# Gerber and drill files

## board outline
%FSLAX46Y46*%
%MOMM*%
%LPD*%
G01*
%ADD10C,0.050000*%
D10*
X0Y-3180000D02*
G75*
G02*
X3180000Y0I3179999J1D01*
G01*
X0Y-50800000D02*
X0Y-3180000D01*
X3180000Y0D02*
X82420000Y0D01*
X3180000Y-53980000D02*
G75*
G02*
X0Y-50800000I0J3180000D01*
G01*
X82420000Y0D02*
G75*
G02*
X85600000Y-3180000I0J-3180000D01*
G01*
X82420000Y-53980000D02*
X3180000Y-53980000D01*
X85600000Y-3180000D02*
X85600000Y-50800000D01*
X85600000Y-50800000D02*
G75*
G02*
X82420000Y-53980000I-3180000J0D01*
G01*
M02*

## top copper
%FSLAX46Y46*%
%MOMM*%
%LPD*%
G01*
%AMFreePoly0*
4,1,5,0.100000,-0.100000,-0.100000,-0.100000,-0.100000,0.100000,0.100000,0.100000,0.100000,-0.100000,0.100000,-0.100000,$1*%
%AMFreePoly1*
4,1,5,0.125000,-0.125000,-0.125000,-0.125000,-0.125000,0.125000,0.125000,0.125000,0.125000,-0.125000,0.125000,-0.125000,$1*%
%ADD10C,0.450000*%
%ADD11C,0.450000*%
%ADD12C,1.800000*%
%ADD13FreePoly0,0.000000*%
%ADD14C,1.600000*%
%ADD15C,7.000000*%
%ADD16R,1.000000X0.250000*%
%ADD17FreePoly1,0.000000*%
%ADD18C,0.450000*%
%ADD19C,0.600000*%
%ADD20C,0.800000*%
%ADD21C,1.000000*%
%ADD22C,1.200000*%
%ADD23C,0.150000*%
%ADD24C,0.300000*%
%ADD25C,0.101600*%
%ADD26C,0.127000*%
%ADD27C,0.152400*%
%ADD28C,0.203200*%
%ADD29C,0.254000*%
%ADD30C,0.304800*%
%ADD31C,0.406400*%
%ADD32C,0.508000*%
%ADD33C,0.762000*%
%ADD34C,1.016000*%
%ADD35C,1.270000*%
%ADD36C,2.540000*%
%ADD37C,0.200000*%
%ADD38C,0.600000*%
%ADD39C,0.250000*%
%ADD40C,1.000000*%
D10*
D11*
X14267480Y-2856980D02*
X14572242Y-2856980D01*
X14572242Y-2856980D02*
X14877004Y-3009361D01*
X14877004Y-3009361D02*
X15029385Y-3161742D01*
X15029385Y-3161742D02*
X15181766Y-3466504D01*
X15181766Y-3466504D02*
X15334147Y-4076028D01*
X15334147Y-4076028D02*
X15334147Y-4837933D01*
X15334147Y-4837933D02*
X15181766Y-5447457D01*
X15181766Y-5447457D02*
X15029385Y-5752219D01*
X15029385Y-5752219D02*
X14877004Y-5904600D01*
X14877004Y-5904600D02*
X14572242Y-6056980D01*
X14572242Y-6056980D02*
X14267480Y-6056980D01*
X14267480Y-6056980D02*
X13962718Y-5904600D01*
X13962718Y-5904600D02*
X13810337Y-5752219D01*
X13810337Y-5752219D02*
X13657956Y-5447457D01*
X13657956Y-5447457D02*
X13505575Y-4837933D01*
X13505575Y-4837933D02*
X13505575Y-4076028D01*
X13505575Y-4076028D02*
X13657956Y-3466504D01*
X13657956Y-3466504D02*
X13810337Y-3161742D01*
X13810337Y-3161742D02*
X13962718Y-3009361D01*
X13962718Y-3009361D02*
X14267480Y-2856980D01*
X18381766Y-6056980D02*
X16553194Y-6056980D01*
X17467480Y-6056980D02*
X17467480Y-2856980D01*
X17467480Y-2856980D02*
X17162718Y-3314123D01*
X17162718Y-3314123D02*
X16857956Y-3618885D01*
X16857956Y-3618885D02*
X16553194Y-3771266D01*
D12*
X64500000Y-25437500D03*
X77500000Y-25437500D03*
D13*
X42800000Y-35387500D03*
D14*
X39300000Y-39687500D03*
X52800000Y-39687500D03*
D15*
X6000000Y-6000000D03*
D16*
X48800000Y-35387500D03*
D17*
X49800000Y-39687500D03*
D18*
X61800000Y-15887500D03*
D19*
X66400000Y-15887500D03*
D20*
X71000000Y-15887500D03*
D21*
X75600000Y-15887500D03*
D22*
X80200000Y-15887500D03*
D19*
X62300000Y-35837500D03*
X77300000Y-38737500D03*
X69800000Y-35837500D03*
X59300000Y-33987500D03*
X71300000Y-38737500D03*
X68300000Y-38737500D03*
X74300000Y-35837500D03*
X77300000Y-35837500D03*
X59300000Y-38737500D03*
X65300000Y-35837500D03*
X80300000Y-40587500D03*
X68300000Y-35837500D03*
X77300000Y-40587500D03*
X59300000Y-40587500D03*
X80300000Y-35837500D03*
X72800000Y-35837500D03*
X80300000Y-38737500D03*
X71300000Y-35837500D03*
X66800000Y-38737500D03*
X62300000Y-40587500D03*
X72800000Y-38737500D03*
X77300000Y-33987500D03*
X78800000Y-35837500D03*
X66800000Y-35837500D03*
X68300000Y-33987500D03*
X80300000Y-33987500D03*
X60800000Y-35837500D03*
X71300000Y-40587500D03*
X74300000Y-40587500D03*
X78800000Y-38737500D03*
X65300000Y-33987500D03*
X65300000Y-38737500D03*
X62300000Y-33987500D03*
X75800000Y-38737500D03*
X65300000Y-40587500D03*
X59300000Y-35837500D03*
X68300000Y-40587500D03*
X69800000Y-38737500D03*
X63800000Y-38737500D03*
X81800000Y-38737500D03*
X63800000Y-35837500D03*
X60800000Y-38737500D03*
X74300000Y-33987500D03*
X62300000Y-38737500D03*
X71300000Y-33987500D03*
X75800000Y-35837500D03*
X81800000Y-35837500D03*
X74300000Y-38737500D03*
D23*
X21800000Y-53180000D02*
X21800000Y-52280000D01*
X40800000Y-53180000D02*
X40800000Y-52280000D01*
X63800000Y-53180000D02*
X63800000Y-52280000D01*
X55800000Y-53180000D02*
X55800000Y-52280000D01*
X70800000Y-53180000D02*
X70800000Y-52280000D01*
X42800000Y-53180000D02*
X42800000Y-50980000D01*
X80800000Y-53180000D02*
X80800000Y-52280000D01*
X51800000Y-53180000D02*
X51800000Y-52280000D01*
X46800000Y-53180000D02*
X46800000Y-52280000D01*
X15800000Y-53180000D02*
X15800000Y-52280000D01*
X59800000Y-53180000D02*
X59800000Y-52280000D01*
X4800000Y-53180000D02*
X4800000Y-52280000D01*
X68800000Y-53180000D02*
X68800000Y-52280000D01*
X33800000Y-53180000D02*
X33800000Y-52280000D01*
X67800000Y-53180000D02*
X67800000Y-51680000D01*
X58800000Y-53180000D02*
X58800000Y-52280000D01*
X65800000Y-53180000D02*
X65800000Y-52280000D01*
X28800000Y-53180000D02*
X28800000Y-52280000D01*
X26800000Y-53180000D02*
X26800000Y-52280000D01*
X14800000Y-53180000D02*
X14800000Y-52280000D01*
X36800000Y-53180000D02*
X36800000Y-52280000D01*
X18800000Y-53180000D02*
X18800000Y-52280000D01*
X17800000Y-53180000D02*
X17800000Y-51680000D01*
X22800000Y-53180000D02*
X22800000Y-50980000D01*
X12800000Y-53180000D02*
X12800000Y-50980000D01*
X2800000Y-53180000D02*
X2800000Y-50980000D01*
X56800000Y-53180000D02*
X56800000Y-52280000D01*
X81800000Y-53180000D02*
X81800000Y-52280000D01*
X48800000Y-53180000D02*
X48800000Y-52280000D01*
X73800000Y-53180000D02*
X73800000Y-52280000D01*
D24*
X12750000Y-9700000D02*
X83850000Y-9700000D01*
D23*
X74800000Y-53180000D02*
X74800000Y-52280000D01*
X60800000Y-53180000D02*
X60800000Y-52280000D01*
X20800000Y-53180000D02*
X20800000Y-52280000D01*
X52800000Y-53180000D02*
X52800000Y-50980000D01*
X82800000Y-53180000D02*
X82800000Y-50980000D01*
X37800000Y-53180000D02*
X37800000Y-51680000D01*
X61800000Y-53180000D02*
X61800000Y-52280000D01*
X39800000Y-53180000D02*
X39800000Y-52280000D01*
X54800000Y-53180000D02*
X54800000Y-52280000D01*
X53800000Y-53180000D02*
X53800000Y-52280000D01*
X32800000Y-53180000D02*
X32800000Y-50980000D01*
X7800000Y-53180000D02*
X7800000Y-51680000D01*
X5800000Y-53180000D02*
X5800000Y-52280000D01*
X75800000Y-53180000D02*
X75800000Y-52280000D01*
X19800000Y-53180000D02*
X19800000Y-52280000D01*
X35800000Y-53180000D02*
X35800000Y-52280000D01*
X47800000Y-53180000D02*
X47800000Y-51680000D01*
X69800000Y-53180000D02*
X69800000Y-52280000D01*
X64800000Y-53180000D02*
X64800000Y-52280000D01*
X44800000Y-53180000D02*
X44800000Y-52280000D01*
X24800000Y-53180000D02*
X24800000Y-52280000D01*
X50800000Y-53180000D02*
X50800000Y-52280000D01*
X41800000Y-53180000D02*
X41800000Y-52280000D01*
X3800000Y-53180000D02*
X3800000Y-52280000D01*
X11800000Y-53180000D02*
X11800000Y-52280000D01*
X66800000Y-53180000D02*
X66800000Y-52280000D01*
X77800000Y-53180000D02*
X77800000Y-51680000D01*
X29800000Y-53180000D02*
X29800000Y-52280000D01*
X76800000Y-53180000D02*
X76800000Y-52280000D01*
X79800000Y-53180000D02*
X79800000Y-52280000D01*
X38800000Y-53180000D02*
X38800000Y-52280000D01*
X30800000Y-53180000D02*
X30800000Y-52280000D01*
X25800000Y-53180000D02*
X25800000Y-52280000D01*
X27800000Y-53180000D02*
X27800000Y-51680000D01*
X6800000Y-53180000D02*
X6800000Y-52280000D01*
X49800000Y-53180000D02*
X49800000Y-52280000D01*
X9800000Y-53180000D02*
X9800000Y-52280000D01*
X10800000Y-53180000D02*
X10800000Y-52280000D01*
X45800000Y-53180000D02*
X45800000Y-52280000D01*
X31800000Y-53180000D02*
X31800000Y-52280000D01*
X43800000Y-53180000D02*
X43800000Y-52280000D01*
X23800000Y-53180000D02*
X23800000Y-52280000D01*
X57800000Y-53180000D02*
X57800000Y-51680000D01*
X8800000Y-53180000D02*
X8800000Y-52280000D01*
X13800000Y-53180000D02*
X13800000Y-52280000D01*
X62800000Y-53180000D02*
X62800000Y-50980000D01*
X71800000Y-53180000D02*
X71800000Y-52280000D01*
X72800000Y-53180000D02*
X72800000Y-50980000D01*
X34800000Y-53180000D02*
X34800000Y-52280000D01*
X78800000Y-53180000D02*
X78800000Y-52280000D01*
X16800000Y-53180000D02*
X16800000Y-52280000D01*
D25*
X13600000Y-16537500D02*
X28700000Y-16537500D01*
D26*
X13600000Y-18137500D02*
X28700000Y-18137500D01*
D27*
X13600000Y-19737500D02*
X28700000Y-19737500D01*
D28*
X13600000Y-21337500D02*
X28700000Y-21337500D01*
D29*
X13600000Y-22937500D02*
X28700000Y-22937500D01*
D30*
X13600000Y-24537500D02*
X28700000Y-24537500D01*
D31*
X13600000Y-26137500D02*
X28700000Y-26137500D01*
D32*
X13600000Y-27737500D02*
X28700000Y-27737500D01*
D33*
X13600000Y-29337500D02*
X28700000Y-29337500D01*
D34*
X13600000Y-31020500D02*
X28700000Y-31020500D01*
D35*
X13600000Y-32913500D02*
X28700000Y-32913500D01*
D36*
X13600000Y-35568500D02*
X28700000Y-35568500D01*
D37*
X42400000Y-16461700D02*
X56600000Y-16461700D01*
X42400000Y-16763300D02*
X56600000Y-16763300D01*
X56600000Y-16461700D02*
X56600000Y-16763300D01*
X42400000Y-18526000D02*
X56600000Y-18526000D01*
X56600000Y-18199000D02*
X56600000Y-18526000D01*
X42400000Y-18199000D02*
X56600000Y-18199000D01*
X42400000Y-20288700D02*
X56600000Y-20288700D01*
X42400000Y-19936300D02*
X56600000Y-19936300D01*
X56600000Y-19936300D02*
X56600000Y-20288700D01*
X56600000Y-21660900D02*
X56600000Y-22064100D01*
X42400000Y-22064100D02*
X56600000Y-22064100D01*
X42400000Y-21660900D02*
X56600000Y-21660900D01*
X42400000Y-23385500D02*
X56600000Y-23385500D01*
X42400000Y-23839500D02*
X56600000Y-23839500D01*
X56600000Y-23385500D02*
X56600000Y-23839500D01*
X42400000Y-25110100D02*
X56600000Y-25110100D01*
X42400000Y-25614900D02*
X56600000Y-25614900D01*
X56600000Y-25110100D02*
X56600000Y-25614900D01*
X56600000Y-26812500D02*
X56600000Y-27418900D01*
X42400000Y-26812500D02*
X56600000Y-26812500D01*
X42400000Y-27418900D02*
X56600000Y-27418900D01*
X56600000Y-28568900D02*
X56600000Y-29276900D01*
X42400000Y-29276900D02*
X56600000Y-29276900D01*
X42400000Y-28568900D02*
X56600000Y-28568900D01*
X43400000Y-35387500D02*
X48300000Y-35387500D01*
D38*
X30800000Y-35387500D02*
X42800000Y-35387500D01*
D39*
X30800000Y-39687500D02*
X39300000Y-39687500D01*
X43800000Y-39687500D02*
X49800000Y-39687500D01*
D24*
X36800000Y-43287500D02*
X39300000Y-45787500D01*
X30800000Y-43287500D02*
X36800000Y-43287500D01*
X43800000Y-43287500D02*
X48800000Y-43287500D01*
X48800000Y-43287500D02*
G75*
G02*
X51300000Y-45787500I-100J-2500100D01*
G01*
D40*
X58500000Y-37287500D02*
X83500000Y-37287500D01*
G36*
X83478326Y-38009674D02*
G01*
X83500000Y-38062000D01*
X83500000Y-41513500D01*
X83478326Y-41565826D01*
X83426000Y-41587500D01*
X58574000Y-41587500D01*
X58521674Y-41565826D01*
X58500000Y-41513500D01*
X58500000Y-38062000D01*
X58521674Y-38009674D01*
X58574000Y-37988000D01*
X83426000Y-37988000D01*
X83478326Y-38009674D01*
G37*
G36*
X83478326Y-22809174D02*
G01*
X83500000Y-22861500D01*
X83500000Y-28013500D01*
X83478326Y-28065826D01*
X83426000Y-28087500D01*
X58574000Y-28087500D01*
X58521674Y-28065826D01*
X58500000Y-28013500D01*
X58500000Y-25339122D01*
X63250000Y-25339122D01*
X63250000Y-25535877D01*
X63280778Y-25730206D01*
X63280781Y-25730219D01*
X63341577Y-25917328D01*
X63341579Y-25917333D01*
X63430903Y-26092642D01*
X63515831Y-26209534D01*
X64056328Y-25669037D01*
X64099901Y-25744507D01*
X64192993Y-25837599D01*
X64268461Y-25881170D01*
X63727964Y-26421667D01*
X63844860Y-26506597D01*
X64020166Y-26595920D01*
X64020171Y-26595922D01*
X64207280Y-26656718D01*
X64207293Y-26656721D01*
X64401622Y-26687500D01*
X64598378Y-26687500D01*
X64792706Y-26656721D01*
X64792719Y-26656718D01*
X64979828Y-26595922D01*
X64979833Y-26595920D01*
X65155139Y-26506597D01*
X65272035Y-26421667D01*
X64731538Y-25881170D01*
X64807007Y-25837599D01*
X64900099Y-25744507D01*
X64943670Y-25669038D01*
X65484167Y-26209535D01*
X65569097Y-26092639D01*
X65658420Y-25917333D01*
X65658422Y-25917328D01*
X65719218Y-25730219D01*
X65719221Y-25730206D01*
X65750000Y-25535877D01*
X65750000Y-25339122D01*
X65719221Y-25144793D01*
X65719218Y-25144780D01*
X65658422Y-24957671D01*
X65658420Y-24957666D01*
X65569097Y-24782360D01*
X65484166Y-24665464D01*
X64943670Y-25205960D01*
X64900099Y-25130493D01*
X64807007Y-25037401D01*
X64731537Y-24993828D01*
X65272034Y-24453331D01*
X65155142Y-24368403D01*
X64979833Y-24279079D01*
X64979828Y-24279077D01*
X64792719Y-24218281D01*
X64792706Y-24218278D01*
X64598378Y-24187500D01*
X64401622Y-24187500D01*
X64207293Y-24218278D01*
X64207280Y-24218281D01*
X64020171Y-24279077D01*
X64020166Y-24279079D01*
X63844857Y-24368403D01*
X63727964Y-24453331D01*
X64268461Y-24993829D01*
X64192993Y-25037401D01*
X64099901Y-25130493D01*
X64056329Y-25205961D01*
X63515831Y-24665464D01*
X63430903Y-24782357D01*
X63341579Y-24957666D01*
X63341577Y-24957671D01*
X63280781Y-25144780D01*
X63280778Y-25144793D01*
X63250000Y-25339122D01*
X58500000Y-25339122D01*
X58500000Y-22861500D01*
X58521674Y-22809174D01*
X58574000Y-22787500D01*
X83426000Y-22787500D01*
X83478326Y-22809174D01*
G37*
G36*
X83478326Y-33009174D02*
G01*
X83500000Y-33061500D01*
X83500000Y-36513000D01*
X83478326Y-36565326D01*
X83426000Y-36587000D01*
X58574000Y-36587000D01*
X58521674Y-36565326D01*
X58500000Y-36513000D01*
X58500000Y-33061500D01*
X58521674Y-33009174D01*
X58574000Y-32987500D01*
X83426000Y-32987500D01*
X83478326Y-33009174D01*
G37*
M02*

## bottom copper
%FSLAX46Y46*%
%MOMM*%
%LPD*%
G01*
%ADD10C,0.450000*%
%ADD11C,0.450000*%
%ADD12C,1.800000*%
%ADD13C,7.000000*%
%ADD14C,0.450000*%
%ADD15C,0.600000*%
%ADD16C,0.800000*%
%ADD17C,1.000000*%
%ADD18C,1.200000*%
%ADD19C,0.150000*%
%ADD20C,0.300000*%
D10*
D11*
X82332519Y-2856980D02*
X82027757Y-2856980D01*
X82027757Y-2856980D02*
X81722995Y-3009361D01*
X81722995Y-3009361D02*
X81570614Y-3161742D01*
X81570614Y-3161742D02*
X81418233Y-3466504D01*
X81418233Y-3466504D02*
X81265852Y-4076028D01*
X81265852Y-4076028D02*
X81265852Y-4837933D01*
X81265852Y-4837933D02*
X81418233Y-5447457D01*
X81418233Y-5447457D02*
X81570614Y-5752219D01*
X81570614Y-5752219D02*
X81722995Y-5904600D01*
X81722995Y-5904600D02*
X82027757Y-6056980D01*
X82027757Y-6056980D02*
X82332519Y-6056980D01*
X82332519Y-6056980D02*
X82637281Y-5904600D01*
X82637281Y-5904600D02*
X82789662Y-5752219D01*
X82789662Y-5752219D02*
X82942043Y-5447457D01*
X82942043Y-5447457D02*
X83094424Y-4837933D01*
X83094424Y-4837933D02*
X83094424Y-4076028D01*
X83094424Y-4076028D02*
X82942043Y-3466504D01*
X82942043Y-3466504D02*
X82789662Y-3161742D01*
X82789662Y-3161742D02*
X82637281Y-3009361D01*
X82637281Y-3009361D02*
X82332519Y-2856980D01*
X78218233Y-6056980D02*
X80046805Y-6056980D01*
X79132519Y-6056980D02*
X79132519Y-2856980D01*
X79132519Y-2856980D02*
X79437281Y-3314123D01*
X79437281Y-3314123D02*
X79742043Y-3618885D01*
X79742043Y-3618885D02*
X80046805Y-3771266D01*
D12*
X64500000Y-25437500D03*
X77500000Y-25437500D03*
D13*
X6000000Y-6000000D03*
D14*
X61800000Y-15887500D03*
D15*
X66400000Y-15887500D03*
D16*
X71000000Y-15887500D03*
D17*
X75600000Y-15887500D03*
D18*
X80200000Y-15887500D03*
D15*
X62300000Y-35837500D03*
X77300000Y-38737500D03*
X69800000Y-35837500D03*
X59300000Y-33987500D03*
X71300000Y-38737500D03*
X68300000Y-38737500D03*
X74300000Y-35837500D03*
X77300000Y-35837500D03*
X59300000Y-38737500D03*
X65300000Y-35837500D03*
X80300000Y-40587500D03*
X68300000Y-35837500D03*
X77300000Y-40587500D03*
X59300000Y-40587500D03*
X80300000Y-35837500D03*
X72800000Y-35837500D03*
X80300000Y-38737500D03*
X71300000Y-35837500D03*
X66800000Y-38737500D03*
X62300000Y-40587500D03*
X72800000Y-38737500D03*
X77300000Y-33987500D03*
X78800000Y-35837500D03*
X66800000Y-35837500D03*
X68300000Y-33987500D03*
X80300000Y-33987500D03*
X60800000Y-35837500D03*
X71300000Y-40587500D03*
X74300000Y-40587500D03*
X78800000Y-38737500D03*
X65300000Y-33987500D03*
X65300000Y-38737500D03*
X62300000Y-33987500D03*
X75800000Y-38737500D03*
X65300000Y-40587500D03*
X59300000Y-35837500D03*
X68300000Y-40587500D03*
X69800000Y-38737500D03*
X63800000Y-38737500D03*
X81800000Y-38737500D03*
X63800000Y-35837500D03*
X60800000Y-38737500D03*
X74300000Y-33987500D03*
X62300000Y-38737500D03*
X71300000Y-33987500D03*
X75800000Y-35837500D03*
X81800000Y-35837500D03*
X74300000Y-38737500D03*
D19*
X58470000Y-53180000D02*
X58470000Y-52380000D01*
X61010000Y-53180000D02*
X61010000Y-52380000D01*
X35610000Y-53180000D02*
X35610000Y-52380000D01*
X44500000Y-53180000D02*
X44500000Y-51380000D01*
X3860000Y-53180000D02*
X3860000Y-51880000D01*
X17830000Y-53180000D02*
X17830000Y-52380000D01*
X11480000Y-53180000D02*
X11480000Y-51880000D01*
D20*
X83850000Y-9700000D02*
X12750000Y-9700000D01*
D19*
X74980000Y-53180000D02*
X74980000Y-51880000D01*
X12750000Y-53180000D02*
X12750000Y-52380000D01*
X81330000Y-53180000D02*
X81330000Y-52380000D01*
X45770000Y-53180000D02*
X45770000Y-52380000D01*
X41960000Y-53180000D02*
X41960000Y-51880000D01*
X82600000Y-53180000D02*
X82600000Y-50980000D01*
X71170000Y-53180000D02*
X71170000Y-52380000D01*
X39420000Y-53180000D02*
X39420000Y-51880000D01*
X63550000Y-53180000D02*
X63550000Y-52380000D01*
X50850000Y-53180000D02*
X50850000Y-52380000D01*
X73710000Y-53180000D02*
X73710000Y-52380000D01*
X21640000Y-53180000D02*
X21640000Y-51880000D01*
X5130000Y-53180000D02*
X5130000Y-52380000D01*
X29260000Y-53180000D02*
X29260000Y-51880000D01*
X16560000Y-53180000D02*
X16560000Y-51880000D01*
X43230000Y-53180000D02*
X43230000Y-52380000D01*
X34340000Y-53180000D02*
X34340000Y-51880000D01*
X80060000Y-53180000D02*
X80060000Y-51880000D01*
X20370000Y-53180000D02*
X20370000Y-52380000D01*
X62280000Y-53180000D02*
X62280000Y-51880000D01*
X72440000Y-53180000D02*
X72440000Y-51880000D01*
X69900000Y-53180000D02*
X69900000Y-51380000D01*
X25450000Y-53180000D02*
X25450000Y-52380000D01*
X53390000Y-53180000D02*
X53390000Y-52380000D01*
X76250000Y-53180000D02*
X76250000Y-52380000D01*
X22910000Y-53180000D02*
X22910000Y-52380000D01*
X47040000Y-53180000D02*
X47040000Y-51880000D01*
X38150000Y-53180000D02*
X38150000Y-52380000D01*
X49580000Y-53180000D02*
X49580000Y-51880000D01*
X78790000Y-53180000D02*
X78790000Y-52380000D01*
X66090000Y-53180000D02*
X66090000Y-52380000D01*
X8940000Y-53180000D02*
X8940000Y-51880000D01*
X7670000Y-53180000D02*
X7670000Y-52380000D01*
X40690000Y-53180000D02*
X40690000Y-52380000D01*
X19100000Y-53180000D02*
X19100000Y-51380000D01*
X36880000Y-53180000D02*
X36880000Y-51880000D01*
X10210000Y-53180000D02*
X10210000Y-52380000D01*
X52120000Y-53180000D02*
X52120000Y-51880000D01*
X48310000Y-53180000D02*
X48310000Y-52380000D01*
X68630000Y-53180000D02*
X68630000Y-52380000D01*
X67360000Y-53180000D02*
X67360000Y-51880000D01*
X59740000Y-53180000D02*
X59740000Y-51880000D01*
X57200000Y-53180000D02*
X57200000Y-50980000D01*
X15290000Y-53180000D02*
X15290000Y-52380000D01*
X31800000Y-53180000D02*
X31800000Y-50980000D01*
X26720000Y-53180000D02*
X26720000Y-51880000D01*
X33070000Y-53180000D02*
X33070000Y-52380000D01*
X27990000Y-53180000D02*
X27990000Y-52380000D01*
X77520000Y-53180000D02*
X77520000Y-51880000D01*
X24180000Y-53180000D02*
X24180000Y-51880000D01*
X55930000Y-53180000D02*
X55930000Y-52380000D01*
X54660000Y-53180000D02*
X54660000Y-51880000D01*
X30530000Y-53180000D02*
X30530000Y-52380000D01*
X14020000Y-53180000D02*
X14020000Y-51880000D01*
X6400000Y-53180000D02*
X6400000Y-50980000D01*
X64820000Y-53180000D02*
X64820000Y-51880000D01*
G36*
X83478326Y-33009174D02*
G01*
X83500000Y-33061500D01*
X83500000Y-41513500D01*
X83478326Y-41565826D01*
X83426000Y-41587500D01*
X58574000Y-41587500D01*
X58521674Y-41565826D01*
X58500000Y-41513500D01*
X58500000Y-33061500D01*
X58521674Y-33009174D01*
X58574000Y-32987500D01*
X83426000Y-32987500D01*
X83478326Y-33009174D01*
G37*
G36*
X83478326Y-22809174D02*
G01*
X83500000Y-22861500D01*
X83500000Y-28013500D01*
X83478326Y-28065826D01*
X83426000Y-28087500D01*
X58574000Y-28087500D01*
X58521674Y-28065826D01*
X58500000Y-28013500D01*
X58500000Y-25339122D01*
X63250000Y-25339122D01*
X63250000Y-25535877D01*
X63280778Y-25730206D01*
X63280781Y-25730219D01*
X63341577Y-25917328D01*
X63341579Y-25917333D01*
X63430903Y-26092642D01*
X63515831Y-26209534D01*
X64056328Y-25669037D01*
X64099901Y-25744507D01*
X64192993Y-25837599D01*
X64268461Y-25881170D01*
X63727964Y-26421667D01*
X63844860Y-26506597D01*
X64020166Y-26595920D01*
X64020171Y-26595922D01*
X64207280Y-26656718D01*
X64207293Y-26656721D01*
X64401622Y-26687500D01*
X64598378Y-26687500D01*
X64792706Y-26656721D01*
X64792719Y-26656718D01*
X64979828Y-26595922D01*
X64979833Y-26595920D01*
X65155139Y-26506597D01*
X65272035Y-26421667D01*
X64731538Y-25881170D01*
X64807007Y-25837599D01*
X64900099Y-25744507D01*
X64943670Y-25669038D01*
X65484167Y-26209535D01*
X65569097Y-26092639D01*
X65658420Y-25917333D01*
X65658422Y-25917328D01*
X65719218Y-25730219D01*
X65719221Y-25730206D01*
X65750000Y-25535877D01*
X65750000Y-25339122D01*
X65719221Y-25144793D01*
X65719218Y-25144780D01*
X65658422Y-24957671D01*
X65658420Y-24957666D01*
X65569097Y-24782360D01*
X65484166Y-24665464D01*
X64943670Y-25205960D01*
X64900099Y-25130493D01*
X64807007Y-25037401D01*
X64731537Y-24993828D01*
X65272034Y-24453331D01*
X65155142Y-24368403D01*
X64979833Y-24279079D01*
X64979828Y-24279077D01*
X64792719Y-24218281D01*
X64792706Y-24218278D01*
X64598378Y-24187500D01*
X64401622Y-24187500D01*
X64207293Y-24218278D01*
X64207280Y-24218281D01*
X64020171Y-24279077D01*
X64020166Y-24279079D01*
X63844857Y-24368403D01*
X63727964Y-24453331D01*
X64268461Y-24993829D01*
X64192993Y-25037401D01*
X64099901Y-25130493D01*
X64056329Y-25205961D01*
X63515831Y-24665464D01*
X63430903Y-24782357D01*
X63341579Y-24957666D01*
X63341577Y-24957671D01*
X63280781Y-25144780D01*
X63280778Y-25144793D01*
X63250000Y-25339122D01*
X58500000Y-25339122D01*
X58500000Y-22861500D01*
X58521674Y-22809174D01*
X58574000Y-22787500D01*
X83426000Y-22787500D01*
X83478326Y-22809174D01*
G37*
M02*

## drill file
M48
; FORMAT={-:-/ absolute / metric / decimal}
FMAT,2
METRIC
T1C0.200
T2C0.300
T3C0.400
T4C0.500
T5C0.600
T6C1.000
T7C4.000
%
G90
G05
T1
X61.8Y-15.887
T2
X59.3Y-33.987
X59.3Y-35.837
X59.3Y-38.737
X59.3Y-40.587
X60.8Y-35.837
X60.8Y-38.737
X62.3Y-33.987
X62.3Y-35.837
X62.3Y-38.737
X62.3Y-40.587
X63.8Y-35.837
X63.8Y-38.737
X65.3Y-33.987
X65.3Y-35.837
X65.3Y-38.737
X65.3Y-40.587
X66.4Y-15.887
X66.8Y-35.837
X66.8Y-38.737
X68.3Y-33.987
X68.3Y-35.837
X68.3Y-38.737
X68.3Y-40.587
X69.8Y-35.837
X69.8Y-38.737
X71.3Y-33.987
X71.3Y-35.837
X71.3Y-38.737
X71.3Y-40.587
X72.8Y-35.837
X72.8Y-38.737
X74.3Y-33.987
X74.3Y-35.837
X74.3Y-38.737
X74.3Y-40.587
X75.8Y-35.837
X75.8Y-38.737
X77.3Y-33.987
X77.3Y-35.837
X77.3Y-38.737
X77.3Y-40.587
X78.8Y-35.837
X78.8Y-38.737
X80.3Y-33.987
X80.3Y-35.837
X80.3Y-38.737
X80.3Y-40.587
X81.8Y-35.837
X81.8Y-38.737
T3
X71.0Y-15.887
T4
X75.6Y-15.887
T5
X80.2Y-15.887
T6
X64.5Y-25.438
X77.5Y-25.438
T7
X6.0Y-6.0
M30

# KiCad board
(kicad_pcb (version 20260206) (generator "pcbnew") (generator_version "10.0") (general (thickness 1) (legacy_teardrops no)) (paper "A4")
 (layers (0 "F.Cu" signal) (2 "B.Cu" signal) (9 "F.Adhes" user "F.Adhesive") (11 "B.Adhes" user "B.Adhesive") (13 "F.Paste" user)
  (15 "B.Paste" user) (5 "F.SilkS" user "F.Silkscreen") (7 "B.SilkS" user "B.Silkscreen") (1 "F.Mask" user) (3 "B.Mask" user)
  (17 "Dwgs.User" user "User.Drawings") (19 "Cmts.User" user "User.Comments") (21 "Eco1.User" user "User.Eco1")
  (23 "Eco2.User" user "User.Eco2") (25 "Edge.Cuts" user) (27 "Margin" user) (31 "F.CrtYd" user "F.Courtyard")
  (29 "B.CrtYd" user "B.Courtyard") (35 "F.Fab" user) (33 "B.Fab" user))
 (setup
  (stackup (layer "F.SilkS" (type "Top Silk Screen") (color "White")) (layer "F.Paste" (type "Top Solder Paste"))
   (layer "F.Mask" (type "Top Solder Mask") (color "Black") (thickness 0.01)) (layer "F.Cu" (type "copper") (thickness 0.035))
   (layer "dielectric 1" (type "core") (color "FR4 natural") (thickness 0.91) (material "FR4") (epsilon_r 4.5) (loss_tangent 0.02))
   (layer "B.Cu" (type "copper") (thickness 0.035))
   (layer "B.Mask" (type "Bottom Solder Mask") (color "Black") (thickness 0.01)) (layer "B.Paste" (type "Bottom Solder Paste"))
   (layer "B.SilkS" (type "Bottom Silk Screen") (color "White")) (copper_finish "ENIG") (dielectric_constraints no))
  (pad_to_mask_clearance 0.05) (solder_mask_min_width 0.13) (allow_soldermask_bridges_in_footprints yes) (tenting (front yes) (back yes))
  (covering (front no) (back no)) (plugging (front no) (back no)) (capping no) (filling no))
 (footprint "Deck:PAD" (layer "F.Cu") (at 64.5 25.4375)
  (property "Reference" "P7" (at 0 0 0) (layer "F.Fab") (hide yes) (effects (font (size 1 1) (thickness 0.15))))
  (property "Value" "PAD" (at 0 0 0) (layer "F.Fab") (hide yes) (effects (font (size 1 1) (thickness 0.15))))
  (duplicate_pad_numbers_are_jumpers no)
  (pad "1" thru_hole circle (at 0 0) (size 1.8 1.8) (drill 1) (layers "*.Cu" "*.Mask") (remove_unused_layers no) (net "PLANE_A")
   (zone_connect 1)))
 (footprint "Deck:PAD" (layer "F.Cu") (at 77.5 25.4375)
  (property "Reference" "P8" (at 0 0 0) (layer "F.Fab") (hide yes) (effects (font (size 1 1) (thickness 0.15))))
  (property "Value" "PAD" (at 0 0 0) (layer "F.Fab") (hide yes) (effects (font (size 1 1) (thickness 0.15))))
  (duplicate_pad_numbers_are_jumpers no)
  (pad "1" thru_hole circle (at 0 0) (size 1.8 1.8) (drill 1) (layers "*.Cu" "*.Mask") (remove_unused_layers no) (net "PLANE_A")
   (zone_connect 2)))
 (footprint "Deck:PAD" (layer "F.Cu") (at 42.8 35.3875)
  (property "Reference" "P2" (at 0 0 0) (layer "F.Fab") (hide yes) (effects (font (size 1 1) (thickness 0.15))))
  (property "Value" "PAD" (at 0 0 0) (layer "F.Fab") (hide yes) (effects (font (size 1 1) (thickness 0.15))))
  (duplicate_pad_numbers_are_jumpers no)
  (pad "1" smd custom (at 0 0) (size 0.2 0.2) (layers "F.Cu" "F.Mask") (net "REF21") (options (clearance outline) (anchor rect))
   (primitives)))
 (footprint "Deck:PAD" (layer "F.Cu") (at 39.3 39.6875)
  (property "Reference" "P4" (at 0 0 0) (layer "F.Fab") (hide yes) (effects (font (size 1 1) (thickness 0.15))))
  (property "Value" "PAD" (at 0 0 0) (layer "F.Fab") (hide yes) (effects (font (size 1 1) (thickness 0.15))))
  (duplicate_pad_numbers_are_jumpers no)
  (pad "1" smd circle (at 0 0) (size 1.6 1.6) (layers "F.Cu" "F.Mask") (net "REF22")))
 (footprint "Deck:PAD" (layer "F.Cu") (at 52.8 39.6875)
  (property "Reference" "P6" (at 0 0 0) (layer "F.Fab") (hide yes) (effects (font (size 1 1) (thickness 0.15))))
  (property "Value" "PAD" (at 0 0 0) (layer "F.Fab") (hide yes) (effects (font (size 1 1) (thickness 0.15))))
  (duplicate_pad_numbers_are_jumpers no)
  (pad "1" smd circle (at 0 0) (size 1.6 1.6) (layers "F.Cu" "F.Mask") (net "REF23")))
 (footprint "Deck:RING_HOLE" (layer "F.Cu") (at 6 6)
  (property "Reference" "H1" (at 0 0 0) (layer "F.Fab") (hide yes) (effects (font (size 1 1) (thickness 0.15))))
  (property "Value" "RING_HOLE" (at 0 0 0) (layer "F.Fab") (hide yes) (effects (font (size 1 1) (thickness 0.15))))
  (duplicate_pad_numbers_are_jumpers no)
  (pad "" thru_hole circle (at 0 0) (size 7 7) (drill 4) (layers "*.Cu" "*.Mask") (remove_unused_layers no)))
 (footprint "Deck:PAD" (layer "F.Cu") (at 48.8 35.3875)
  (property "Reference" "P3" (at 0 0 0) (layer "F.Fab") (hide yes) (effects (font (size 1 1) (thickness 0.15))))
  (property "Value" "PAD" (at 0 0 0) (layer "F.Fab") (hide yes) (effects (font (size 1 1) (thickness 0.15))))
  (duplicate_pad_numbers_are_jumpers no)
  (pad "1" smd rect (at 0 0) (size 1 0.25) (layers "F.Cu" "F.Mask") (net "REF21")))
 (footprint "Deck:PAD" (layer "F.Cu") (at 49.8 39.6875)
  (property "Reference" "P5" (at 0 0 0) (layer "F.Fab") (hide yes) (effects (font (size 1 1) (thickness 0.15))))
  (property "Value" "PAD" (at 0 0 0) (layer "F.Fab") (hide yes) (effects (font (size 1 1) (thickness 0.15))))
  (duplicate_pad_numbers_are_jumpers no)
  (pad "1" smd custom (at 0 0) (size 0.25 0.25) (layers "F.Cu" "F.Mask") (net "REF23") (options (clearance outline) (anchor rect))
   (primitives)))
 (gr_arc (start 0 3.18) (mid 0.9314 0.9314) (end 3.18 0) (stroke (width 0.05) (type solid)) (layer "Edge.Cuts"))
 (gr_line (start 0 50.8) (end 0 3.18) (stroke (width 0.05) (type solid)) (layer "Edge.Cuts"))
 (gr_line (start 3.18 0) (end 82.42 0) (stroke (width 0.05) (type solid)) (layer "Edge.Cuts"))
 (gr_arc (start 3.18 53.98) (mid 0.9314 53.0486) (end 0 50.8) (stroke (width 0.05) (type solid)) (layer "Edge.Cuts"))
 (gr_arc (start 82.42 0) (mid 84.6686 0.9314) (end 85.6 3.18) (stroke (width 0.05) (type solid)) (layer "Edge.Cuts"))
 (gr_line (start 82.42 53.98) (end 3.18 53.98) (stroke (width 0.05) (type solid)) (layer "Edge.Cuts"))
 (gr_line (start 85.6 3.18) (end 85.6 50.8) (stroke (width 0.05) (type solid)) (layer "Edge.Cuts"))
 (gr_arc (start 85.6 50.8) (mid 84.6686 53.0486) (end 82.42 53.98) (stroke (width 0.05) (type solid)) (layer "Edge.Cuts"))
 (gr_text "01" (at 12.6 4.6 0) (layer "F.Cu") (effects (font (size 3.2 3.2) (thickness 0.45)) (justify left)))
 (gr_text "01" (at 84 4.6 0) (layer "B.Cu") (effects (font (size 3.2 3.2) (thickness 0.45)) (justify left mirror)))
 (segment (start 21.8 53.18) (end 21.8 52.28) (width 0.15) (layer "F.Cu") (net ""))
 (segment (start 40.8 53.18) (end 40.8 52.28) (width 0.15) (layer "F.Cu") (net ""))
 (segment (start 63.8 53.18) (end 63.8 52.28) (width 0.15) (layer "F.Cu") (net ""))
 (segment (start 55.8 53.18) (end 55.8 52.28) (width 0.15) (layer "F.Cu") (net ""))
 (segment (start 70.8 53.18) (end 70.8 52.28) (width 0.15) (layer "F.Cu") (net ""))
 (segment (start 42.8 53.18) (end 42.8 50.98) (width 0.15) (layer "F.Cu") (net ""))
 (segment (start 80.8 53.18) (end 80.8 52.28) (width 0.15) (layer "F.Cu") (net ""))
 (segment (start 51.8 53.18) (end 51.8 52.28) (width 0.15) (layer "F.Cu") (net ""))
 (segment (start 46.8 53.18) (end 46.8 52.28) (width 0.15) (layer "F.Cu") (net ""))
 (segment (start 15.8 53.18) (end 15.8 52.28) (width 0.15) (layer "F.Cu") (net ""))
 (segment (start 59.8 53.18) (end 59.8 52.28) (width 0.15) (layer "F.Cu") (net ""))
 (segment (start 4.8 53.18) (end 4.8 52.28) (width 0.15) (layer "F.Cu") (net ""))
 (segment (start 68.8 53.18) (end 68.8 52.28) (width 0.15) (layer "F.Cu") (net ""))
 (segment (start 33.8 53.18) (end 33.8 52.28) (width 0.15) (layer "F.Cu") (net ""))
 (segment (start 67.8 53.18) (end 67.8 51.68) (width 0.15) (layer "F.Cu") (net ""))
 (segment (start 58.8 53.18) (end 58.8 52.28) (width 0.15) (layer "F.Cu") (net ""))
 (segment (start 65.8 53.18) (end 65.8 52.28) (width 0.15) (layer "F.Cu") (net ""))
 (segment (start 28.8 53.18) (end 28.8 52.28) (width 0.15) (layer "F.Cu") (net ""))
 (segment (start 26.8 53.18) (end 26.8 52.28) (width 0.15) (layer "F.Cu") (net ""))
 (segment (start 14.8 53.18) (end 14.8 52.28) (width 0.15) (layer "F.Cu") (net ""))
 (segment (start 36.8 53.18) (end 36.8 52.28) (width 0.15) (layer "F.Cu") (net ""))
 (segment (start 18.8 53.18) (end 18.8 52.28) (width 0.15) (layer "F.Cu") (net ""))
 (segment (start 17.8 53.18) (end 17.8 51.68) (width 0.15) (layer "F.Cu") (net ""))
 (segment (start 22.8 53.18) (end 22.8 50.98) (width 0.15) (layer "F.Cu") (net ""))
 (segment (start 12.8 53.18) (end 12.8 50.98) (width 0.15) (layer "F.Cu") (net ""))
 (segment (start 2.8 53.18) (end 2.8 50.98) (width 0.15) (layer "F.Cu") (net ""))
 (segment (start 56.8 53.18) (end 56.8 52.28) (width 0.15) (layer "F.Cu") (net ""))
 (segment (start 81.8 53.18) (end 81.8 52.28) (width 0.15) (layer "F.Cu") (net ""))
 (segment (start 48.8 53.18) (end 48.8 52.28) (width 0.15) (layer "F.Cu") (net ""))
 (segment (start 73.8 53.18) (end 73.8 52.28) (width 0.15) (layer "F.Cu") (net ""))
 (segment (start 12.75 9.7) (end 83.85 9.7) (width 0.3) (layer "F.Cu") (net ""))
 (segment (start 74.8 53.18) (end 74.8 52.28) (width 0.15) (layer "F.Cu") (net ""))
 (segment (start 60.8 53.18) (end 60.8 52.28) (width 0.15) (layer "F.Cu") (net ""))
 (segment (start 20.8 53.18) (end 20.8 52.28) (width 0.15) (layer "F.Cu") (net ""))
 (segment (start 52.8 53.18) (end 52.8 50.98) (width 0.15) (layer "F.Cu") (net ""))
 (segment (start 82.8 53.18) (end 82.8 50.98) (width 0.15) (layer "F.Cu") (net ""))
 (segment (start 37.8 53.18) (end 37.8 51.68) (width 0.15) (layer "F.Cu") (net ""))
 (segment (start 61.8 53.18) (end 61.8 52.28) (width 0.15) (layer "F.Cu") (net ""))
 (segment (start 39.8 53.18) (end 39.8 52.28) (width 0.15) (layer "F.Cu") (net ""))
 (segment (start 54.8 53.18) (end 54.8 52.28) (width 0.15) (layer "F.Cu") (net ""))
 (segment (start 53.8 53.18) (end 53.8 52.28) (width 0.15) (layer "F.Cu") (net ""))
 (segment (start 32.8 53.18) (end 32.8 50.98) (width 0.15) (layer "F.Cu") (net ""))
 (segment (start 7.8 53.18) (end 7.8 51.68) (width 0.15) (layer "F.Cu") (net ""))
 (segment (start 5.8 53.18) (end 5.8 52.28) (width 0.15) (layer "F.Cu") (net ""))
 (segment (start 75.8 53.18) (end 75.8 52.28) (width 0.15) (layer "F.Cu") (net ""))
 (segment (start 19.8 53.18) (end 19.8 52.28) (width 0.15) (layer "F.Cu") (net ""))
 (segment (start 35.8 53.18) (end 35.8 52.28) (width 0.15) (layer "F.Cu") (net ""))
 (segment (start 47.8 53.18) (end 47.8 51.68) (width 0.15) (layer "F.Cu") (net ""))
 (segment (start 69.8 53.18) (end 69.8 52.28) (width 0.15) (layer "F.Cu") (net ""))
 (segment (start 64.8 53.18) (end 64.8 52.28) (width 0.15) (layer "F.Cu") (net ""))
 (segment (start 44.8 53.18) (end 44.8 52.28) (width 0.15) (layer "F.Cu") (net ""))
 (segment (start 24.8 53.18) (end 24.8 52.28) (width 0.15) (layer "F.Cu") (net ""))
 (segment (start 50.8 53.18) (end 50.8 52.28) (width 0.15) (layer "F.Cu") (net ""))
 (segment (start 41.8 53.18) (end 41.8 52.28) (width 0.15) (layer "F.Cu") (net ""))
 (segment (start 3.8 53.18) (end 3.8 52.28) (width 0.15) (layer "F.Cu") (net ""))
 (segment (start 11.8 53.18) (end 11.8 52.28) (width 0.15) (layer "F.Cu") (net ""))
 (segment (start 66.8 53.18) (end 66.8 52.28) (width 0.15) (layer "F.Cu") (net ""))
 (segment (start 77.8 53.18) (end 77.8 51.68) (width 0.15) (layer "F.Cu") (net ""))
 (segment (start 29.8 53.18) (end 29.8 52.28) (width 0.15) (layer "F.Cu") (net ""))
 (segment (start 76.8 53.18) (end 76.8 52.28) (width 0.15) (layer "F.Cu") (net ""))
 (segment (start 79.8 53.18) (end 79.8 52.28) (width 0.15) (layer "F.Cu") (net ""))
 (segment (start 38.8 53.18) (end 38.8 52.28) (width 0.15) (layer "F.Cu") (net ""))
 (segment (start 30.8 53.18) (end 30.8 52.28) (width 0.15) (layer "F.Cu") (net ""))
 (segment (start 25.8 53.18) (end 25.8 52.28) (width 0.15) (layer "F.Cu") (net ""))
 (segment (start 27.8 53.18) (end 27.8 51.68) (width 0.15) (layer "F.Cu") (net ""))
 (segment (start 6.8 53.18) (end 6.8 52.28) (width 0.15) (layer "F.Cu") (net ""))
 (segment (start 49.8 53.18) (end 49.8 52.28) (width 0.15) (layer "F.Cu") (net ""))
 (segment (start 9.8 53.18) (end 9.8 52.28) (width 0.15) (layer "F.Cu") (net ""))
 (segment (start 10.8 53.18) (end 10.8 52.28) (width 0.15) (layer "F.Cu") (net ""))
 (segment (start 45.8 53.18) (end 45.8 52.28) (width 0.15) (layer "F.Cu") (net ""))
 (segment (start 31.8 53.18) (end 31.8 52.28) (width 0.15) (layer "F.Cu") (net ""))
 (segment (start 43.8 53.18) (end 43.8 52.28) (width 0.15) (layer "F.Cu") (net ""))
 (segment (start 23.8 53.18) (end 23.8 52.28) (width 0.15) (layer "F.Cu") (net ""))
 (segment (start 57.8 53.18) (end 57.8 51.68) (width 0.15) (layer "F.Cu") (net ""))
 (segment (start 8.8 53.18) (end 8.8 52.28) (width 0.15) (layer "F.Cu") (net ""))
 (segment (start 13.8 53.18) (end 13.8 52.28) (width 0.15) (layer "F.Cu") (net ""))
 (segment (start 62.8 53.18) (end 62.8 50.98) (width 0.15) (layer "F.Cu") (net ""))
 (segment (start 71.8 53.18) (end 71.8 52.28) (width 0.15) (layer "F.Cu") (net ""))
 (segment (start 72.8 53.18) (end 72.8 50.98) (width 0.15) (layer "F.Cu") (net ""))
 (segment (start 34.8 53.18) (end 34.8 52.28) (width 0.15) (layer "F.Cu") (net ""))
 (segment (start 78.8 53.18) (end 78.8 52.28) (width 0.15) (layer "F.Cu") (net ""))
 (segment (start 16.8 53.18) (end 16.8 52.28) (width 0.15) (layer "F.Cu") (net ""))
 (segment (start 58.47 53.18) (end 58.47 52.38) (width 0.15) (layer "B.Cu") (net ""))
 (segment (start 61.01 53.18) (end 61.01 52.38) (width 0.15) (layer "B.Cu") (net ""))
 (segment (start 35.61 53.18) (end 35.61 52.38) (width 0.15) (layer "B.Cu") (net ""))
 (segment (start 44.5 53.18) (end 44.5 51.38) (width 0.15) (layer "B.Cu") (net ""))
 (segment (start 3.86 53.18) (end 3.86 51.88) (width 0.15) (layer "B.Cu") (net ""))
 (segment (start 17.83 53.18) (end 17.83 52.38) (width 0.15) (layer "B.Cu") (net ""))
 (segment (start 11.48 53.18) (end 11.48 51.88) (width 0.15) (layer "B.Cu") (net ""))
 (segment (start 83.85 9.7) (end 12.75 9.7) (width 0.3) (layer "B.Cu") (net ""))
 (segment (start 74.98 53.18) (end 74.98 51.88) (width 0.15) (layer "B.Cu") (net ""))
 (segment (start 12.75 53.18) (end 12.75 52.38) (width 0.15) (layer "B.Cu") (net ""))
 (segment (start 81.33 53.18) (end 81.33 52.38) (width 0.15) (layer "B.Cu") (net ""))
 (segment (start 45.77 53.18) (end 45.77 52.38) (width 0.15) (layer "B.Cu") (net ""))
 (segment (start 41.96 53.18) (end 41.96 51.88) (width 0.15) (layer "B.Cu") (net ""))
 (segment (start 82.6 53.18) (end 82.6 50.98) (width 0.15) (layer "B.Cu") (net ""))
 (segment (start 71.17 53.18) (end 71.17 52.38) (width 0.15) (layer "B.Cu") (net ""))
 (segment (start 39.42 53.18) (end 39.42 51.88) (width 0.15) (layer "B.Cu") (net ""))
 (segment (start 63.55 53.18) (end 63.55 52.38) (width 0.15) (layer "B.Cu") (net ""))
 (segment (start 50.85 53.18) (end 50.85 52.38) (width 0.15) (layer "B.Cu") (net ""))
 (segment (start 73.71 53.18) (end 73.71 52.38) (width 0.15) (layer "B.Cu") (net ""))
 (segment (start 21.64 53.18) (end 21.64 51.88) (width 0.15) (layer "B.Cu") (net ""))
 (segment (start 5.13 53.18) (end 5.13 52.38) (width 0.15) (layer "B.Cu") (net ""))
 (segment (start 29.26 53.18) (end 29.26 51.88) (width 0.15) (layer "B.Cu") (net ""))
 (segment (start 16.56 53.18) (end 16.56 51.88) (width 0.15) (layer "B.Cu") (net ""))
 (segment (start 43.23 53.18) (end 43.23 52.38) (width 0.15) (layer "B.Cu") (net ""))
 (segment (start 34.34 53.18) (end 34.34 51.88) (width 0.15) (layer "B.Cu") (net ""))
 (segment (start 80.06 53.18) (end 80.06 51.88) (width 0.15) (layer "B.Cu") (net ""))
 (segment (start 20.37 53.18) (end 20.37 52.38) (width 0.15) (layer "B.Cu") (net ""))
 (segment (start 62.28 53.18) (end 62.28 51.88) (width 0.15) (layer "B.Cu") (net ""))
 (segment (start 72.44 53.18) (end 72.44 51.88) (width 0.15) (layer "B.Cu") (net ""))
 (segment (start 69.9 53.18) (end 69.9 51.38) (width 0.15) (layer "B.Cu") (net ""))
 (segment (start 25.45 53.18) (end 25.45 52.38) (width 0.15) (layer "B.Cu") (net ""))
 (segment (start 53.39 53.18) (end 53.39 52.38) (width 0.15) (layer "B.Cu") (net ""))
 (segment (start 76.25 53.18) (end 76.25 52.38) (width 0.15) (layer "B.Cu") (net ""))
 (segment (start 22.91 53.18) (end 22.91 52.38) (width 0.15) (layer "B.Cu") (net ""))
 (segment (start 47.04 53.18) (end 47.04 51.88) (width 0.15) (layer "B.Cu") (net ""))
 (segment (start 38.15 53.18) (end 38.15 52.38) (width 0.15) (layer "B.Cu") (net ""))
 (segment (start 49.58 53.18) (end 49.58 51.88) (width 0.15) (layer "B.Cu") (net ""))
 (segment (start 78.79 53.18) (end 78.79 52.38) (width 0.15) (layer "B.Cu") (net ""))
 (segment (start 66.09 53.18) (end 66.09 52.38) (width 0.15) (layer "B.Cu") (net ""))
 (segment (start 8.94 53.18) (end 8.94 51.88) (width 0.15) (layer "B.Cu") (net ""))
 (segment (start 7.67 53.18) (end 7.67 52.38) (width 0.15) (layer "B.Cu") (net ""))
 (segment (start 40.69 53.18) (end 40.69 52.38) (width 0.15) (layer "B.Cu") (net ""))
 (segment (start 19.1 53.18) (end 19.1 51.38) (width 0.15) (layer "B.Cu") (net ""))
 (segment (start 36.88 53.18) (end 36.88 51.88) (width 0.15) (layer "B.Cu") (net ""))
 (segment (start 10.21 53.18) (end 10.21 52.38) (width 0.15) (layer "B.Cu") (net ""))
 (segment (start 52.12 53.18) (end 52.12 51.88) (width 0.15) (layer "B.Cu") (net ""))
 (segment (start 48.31 53.18) (end 48.31 52.38) (width 0.15) (layer "B.Cu") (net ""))
 (segment (start 68.63 53.18) (end 68.63 52.38) (width 0.15) (layer "B.Cu") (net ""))
 (segment (start 67.36 53.18) (end 67.36 51.88) (width 0.15) (layer "B.Cu") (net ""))
 (segment (start 59.74 53.18) (end 59.74 51.88) (width 0.15) (layer "B.Cu") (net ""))
 (segment (start 57.2 53.18) (end 57.2 50.98) (width 0.15) (layer "B.Cu") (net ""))
 (segment (start 15.29 53.18) (end 15.29 52.38) (width 0.15) (layer "B.Cu") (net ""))
 (segment (start 31.8 53.18) (end 31.8 50.98) (width 0.15) (layer "B.Cu") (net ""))
 (segment (start 26.72 53.18) (end 26.72 51.88) (width 0.15) (layer "B.Cu") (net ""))
 (segment (start 33.07 53.18) (end 33.07 52.38) (width 0.15) (layer "B.Cu") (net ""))
 (segment (start 27.99 53.18) (end 27.99 52.38) (width 0.15) (layer "B.Cu") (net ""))
 (segment (start 77.52 53.18) (end 77.52 51.88) (width 0.15) (layer "B.Cu") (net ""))
 (segment (start 24.18 53.18) (end 24.18 51.88) (width 0.15) (layer "B.Cu") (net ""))
 (segment (start 55.93 53.18) (end 55.93 52.38) (width 0.15) (layer "B.Cu") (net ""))
 (segment (start 54.66 53.18) (end 54.66 51.88) (width 0.15) (layer "B.Cu") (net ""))
 (segment (start 30.53 53.18) (end 30.53 52.38) (width 0.15) (layer "B.Cu") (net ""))
 (segment (start 14.02 53.18) (end 14.02 51.88) (width 0.15) (layer "B.Cu") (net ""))
 (segment (start 6.4 53.18) (end 6.4 50.98) (width 0.15) (layer "B.Cu") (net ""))
 (segment (start 64.82 53.18) (end 64.82 51.88) (width 0.15) (layer "B.Cu") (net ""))
 (segment (start 13.6 16.5375) (end 28.7 16.5375) (width 0.1016) (layer "F.Cu") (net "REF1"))
 (segment (start 13.6 18.1375) (end 28.7 18.1375) (width 0.127) (layer "F.Cu") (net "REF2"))
 (segment (start 13.6 19.7375) (end 28.7 19.7375) (width 0.1524) (layer "F.Cu") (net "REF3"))
 (segment (start 13.6 21.3375) (end 28.7 21.3375) (width 0.2032) (layer "F.Cu") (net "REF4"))
 (segment (start 13.6 22.9375) (end 28.7 22.9375) (width 0.254) (layer "F.Cu") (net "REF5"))
 (segment (start 13.6 24.5375) (end 28.7 24.5375) (width 0.3048) (layer "F.Cu") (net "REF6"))
 (segment (start 13.6 26.1375) (end 28.7 26.1375) (width 0.4064) (layer "F.Cu") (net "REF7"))
 (segment (start 13.6 27.7375) (end 28.7 27.7375) (width 0.508) (layer "F.Cu") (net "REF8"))
 (segment (start 13.6 29.3375) (end 28.7 29.3375) (width 0.762) (layer "F.Cu") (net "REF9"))
 (segment (start 13.6 31.0205) (end 28.7 31.0205) (width 1.016) (layer "F.Cu") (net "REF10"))
 (segment (start 13.6 32.9135) (end 28.7 32.9135) (width 1.27) (layer "F.Cu") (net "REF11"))
 (segment (start 13.6 35.5685) (end 28.7 35.5685) (width 2.54) (layer "F.Cu") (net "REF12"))
 (segment (start 42.4 16.4617) (end 56.6 16.4617) (width 0.2) (layer "F.Cu") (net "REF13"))
 (segment (start 42.4 16.7633) (end 56.6 16.7633) (width 0.2) (layer "F.Cu") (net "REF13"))
 (segment (start 56.6 16.4617) (end 56.6 16.7633) (width 0.2) (layer "F.Cu") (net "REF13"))
 (segment (start 42.4 18.526) (end 56.6 18.526) (width 0.2) (layer "F.Cu") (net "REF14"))
 (segment (start 56.6 18.199) (end 56.6 18.526) (width 0.2) (layer "F.Cu") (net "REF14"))
 (segment (start 42.4 18.199) (end 56.6 18.199) (width 0.2) (layer "F.Cu") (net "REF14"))
 (segment (start 42.4 20.2887) (end 56.6 20.2887) (width 0.2) (layer "F.Cu") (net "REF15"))
 (segment (start 42.4 19.9363) (end 56.6 19.9363) (width 0.2) (layer "F.Cu") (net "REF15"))
 (segment (start 56.6 19.9363) (end 56.6 20.2887) (width 0.2) (layer "F.Cu") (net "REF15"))
 (segment (start 56.6 21.6609) (end 56.6 22.0641) (width 0.2) (layer "F.Cu") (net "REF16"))
 (segment (start 42.4 22.0641) (end 56.6 22.0641) (width 0.2) (layer "F.Cu") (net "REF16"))
 (segment (start 42.4 21.6609) (end 56.6 21.6609) (width 0.2) (layer "F.Cu") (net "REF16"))
 (segment (start 42.4 23.3855) (end 56.6 23.3855) (width 0.2) (layer "F.Cu") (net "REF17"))
 (segment (start 42.4 23.8395) (end 56.6 23.8395) (width 0.2) (layer "F.Cu") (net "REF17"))
 (segment (start 56.6 23.3855) (end 56.6 23.8395) (width 0.2) (layer "F.Cu") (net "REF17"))
 (segment (start 42.4 25.1101) (end 56.6 25.1101) (width 0.2) (layer "F.Cu") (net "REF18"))
 (segment (start 42.4 25.6149) (end 56.6 25.6149) (width 0.2) (layer "F.Cu") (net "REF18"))
 (segment (start 56.6 25.1101) (end 56.6 25.6149) (width 0.2) (layer "F.Cu") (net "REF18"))
 (segment (start 56.6 26.8125) (end 56.6 27.4189) (width 0.2) (layer "F.Cu") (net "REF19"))
 (segment (start 42.4 26.8125) (end 56.6 26.8125) (width 0.2) (layer "F.Cu") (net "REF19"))
 (segment (start 42.4 27.4189) (end 56.6 27.4189) (width 0.2) (layer "F.Cu") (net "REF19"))
 (segment (start 56.6 28.5689) (end 56.6 29.2769) (width 0.2) (layer "F.Cu") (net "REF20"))
 (segment (start 42.4 29.2769) (end 56.6 29.2769) (width 0.2) (layer "F.Cu") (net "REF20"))
 (segment (start 42.4 28.5689) (end 56.6 28.5689) (width 0.2) (layer "F.Cu") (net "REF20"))
 (segment (start 43.4 35.3875) (end 48.3 35.3875) (width 0.2) (layer "F.Cu") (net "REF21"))
 (segment (start 30.8 35.3875) (end 42.8 35.3875) (width 0.6) (layer "F.Cu") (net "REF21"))
 (segment (start 30.8 39.6875) (end 39.3 39.6875) (width 0.25) (layer "F.Cu") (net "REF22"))
 (segment (start 43.8 39.6875) (end 49.8 39.6875) (width 0.25) (layer "F.Cu") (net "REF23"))
 (segment (start 36.8 43.2875) (end 39.3 45.7875) (width 0.3) (layer "F.Cu") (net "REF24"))
 (segment (start 30.8 43.2875) (end 36.8 43.2875) (width 0.3) (layer "F.Cu") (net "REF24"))
 (segment (start 43.8 43.2875) (end 48.8 43.2875) (width 0.3) (layer "F.Cu") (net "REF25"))
 (arc (start 48.8 43.2875) (mid 50.56775 44.01975) (end 51.3 45.7875) (width 0.3) (layer "F.Cu") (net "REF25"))
 (via (at 61.8 15.8875) (size 0.45) (drill 0.2) (layers "F.Cu" "B.Cu") (tenting (front no) (back no)) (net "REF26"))
 (via (at 66.4 15.8875) (size 0.6) (drill 0.3) (layers "F.Cu" "B.Cu") (tenting (front no) (back no)) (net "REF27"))
 (via (at 71 15.8875) (size 0.8) (drill 0.4) (layers "F.Cu" "B.Cu") (tenting (front no) (back no)) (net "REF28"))
 (via (at 75.6 15.8875) (size 1) (drill 0.5) (layers "F.Cu" "B.Cu") (tenting (front no) (back no)) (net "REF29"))
 (via (at 80.2 15.8875) (size 1.2) (drill 0.6) (layers "F.Cu" "B.Cu") (tenting (front no) (back no)) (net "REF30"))
 (segment (start 58.5 37.2875) (end 83.5 37.2875) (width 1) (layer "F.Cu") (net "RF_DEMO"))
 (via (at 62.3 35.8375) (size 0.6) (drill 0.3) (layers "F.Cu" "B.Cu") (tenting (front no) (back no)) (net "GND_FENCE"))
 (via (at 77.3 38.7375) (size 0.6) (drill 0.3) (layers "F.Cu" "B.Cu") (tenting (front no) (back no)) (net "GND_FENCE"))
 (via (at 69.8 35.8375) (size 0.6) (drill 0.3) (layers "F.Cu" "B.Cu") (tenting (front no) (back no)) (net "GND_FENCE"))
 (via (at 59.3 33.9875) (size 0.6) (drill 0.3) (layers "F.Cu" "B.Cu") (tenting (front no) (back no)) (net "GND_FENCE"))
 (via (at 71.3 38.7375) (size 0.6) (drill 0.3) (layers "F.Cu" "B.Cu") (tenting (front no) (back no)) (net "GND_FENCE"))
 (via (at 68.3 38.7375) (size 0.6) (drill 0.3) (layers "F.Cu" "B.Cu") (tenting (front no) (back no)) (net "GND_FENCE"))
 (via (at 74.3 35.8375) (size 0.6) (drill 0.3) (layers "F.Cu" "B.Cu") (tenting (front no) (back no)) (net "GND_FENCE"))
 (via (at 77.3 35.8375) (size 0.6) (drill 0.3) (layers "F.Cu" "B.Cu") (tenting (front no) (back no)) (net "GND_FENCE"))
 (via (at 59.3 38.7375) (size 0.6) (drill 0.3) (layers "F.Cu" "B.Cu") (tenting (front no) (back no)) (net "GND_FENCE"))
 (via (at 65.3 35.8375) (size 0.6) (drill 0.3) (layers "F.Cu" "B.Cu") (tenting (front no) (back no)) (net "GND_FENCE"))
 (via (at 80.3 40.5875) (size 0.6) (drill 0.3) (layers "F.Cu" "B.Cu") (tenting (front no) (back no)) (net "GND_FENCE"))
 (via (at 68.3 35.8375) (size 0.6) (drill 0.3) (layers "F.Cu" "B.Cu") (tenting (front no) (back no)) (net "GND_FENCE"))
 (via (at 77.3 40.5875) (size 0.6) (drill 0.3) (layers "F.Cu" "B.Cu") (tenting (front no) (back no)) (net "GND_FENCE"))
 (via (at 59.3 40.5875) (size 0.6) (drill 0.3) (layers "F.Cu" "B.Cu") (tenting (front no) (back no)) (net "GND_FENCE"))
 (via (at 80.3 35.8375) (size 0.6) (drill 0.3) (layers "F.Cu" "B.Cu") (tenting (front no) (back no)) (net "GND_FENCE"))
 (via (at 72.8 35.8375) (size 0.6) (drill 0.3) (layers "F.Cu" "B.Cu") (tenting (front no) (back no)) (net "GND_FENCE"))
 (via (at 80.3 38.7375) (size 0.6) (drill 0.3) (layers "F.Cu" "B.Cu") (tenting (front no) (back no)) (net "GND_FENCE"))
 (via (at 71.3 35.8375) (size 0.6) (drill 0.3) (layers "F.Cu" "B.Cu") (tenting (front no) (back no)) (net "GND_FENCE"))
 (via (at 66.8 38.7375) (size 0.6) (drill 0.3) (layers "F.Cu" "B.Cu") (tenting (front no) (back no)) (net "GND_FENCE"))
 (via (at 62.3 40.5875) (size 0.6) (drill 0.3) (layers "F.Cu" "B.Cu") (tenting (front no) (back no)) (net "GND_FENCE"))
 (via (at 72.8 38.7375) (size 0.6) (drill 0.3) (layers "F.Cu" "B.Cu") (tenting (front no) (back no)) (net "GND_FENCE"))
 (via (at 77.3 33.9875) (size 0.6) (drill 0.3) (layers "F.Cu" "B.Cu") (tenting (front no) (back no)) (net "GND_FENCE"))
 (via (at 78.8 35.8375) (size 0.6) (drill 0.3) (layers "F.Cu" "B.Cu") (tenting (front no) (back no)) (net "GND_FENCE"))
 (via (at 66.8 35.8375) (size 0.6) (drill 0.3) (layers "F.Cu" "B.Cu") (tenting (front no) (back no)) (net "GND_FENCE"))
 (via (at 68.3 33.9875) (size 0.6) (drill 0.3) (layers "F.Cu" "B.Cu") (tenting (front no) (back no)) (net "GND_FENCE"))
 (via (at 80.3 33.9875) (size 0.6) (drill 0.3) (layers "F.Cu" "B.Cu") (tenting (front no) (back no)) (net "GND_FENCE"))
 (via (at 60.8 35.8375) (size 0.6) (drill 0.3) (layers "F.Cu" "B.Cu") (tenting (front no) (back no)) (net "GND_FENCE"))
 (via (at 71.3 40.5875) (size 0.6) (drill 0.3) (layers "F.Cu" "B.Cu") (tenting (front no) (back no)) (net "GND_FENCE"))
 (via (at 74.3 40.5875) (size 0.6) (drill 0.3) (layers "F.Cu" "B.Cu") (tenting (front no) (back no)) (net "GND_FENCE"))
 (via (at 78.8 38.7375) (size 0.6) (drill 0.3) (layers "F.Cu" "B.Cu") (tenting (front no) (back no)) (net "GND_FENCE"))
 (via (at 65.3 33.9875) (size 0.6) (drill 0.3) (layers "F.Cu" "B.Cu") (tenting (front no) (back no)) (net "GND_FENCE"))
 (via (at 65.3 38.7375) (size 0.6) (drill 0.3) (layers "F.Cu" "B.Cu") (tenting (front no) (back no)) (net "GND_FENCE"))
 (via (at 62.3 33.9875) (size 0.6) (drill 0.3) (layers "F.Cu" "B.Cu") (tenting (front no) (back no)) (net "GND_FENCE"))
 (via (at 75.8 38.7375) (size 0.6) (drill 0.3) (layers "F.Cu" "B.Cu") (tenting (front no) (back no)) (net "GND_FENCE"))
 (via (at 65.3 40.5875) (size 0.6) (drill 0.3) (layers "F.Cu" "B.Cu") (tenting (front no) (back no)) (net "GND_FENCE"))
 (via (at 59.3 35.8375) (size 0.6) (drill 0.3) (layers "F.Cu" "B.Cu") (tenting (front no) (back no)) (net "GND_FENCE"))
 (via (at 68.3 40.5875) (size 0.6) (drill 0.3) (layers "F.Cu" "B.Cu") (tenting (front no) (back no)) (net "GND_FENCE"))
 (via (at 69.8 38.7375) (size 0.6) (drill 0.3) (layers "F.Cu" "B.Cu") (tenting (front no) (back no)) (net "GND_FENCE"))
 (via (at 63.8 38.7375) (size 0.6) (drill 0.3) (layers "F.Cu" "B.Cu") (tenting (front no) (back no)) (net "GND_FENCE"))
 (via (at 81.8 38.7375) (size 0.6) (drill 0.3) (layers "F.Cu" "B.Cu") (tenting (front no) (back no)) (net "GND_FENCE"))
 (via (at 63.8 35.8375) (size 0.6) (drill 0.3) (layers "F.Cu" "B.Cu") (tenting (front no) (back no)) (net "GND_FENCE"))
 (via (at 60.8 38.7375) (size 0.6) (drill 0.3) (layers "F.Cu" "B.Cu") (tenting (front no) (back no)) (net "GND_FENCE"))
 (via (at 74.3 33.9875) (size 0.6) (drill 0.3) (layers "F.Cu" "B.Cu") (tenting (front no) (back no)) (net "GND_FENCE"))
 (via (at 62.3 38.7375) (size 0.6) (drill 0.3) (layers "F.Cu" "B.Cu") (tenting (front no) (back no)) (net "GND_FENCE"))
 (via (at 71.3 33.9875) (size 0.6) (drill 0.3) (layers "F.Cu" "B.Cu") (tenting (front no) (back no)) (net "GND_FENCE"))
 (via (at 75.8 35.8375) (size 0.6) (drill 0.3) (layers "F.Cu" "B.Cu") (tenting (front no) (back no)) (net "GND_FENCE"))
 (via (at 81.8 35.8375) (size 0.6) (drill 0.3) (layers "F.Cu" "B.Cu") (tenting (front no) (back no)) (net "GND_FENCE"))
 (via (at 74.3 38.7375) (size 0.6) (drill 0.3) (layers "F.Cu" "B.Cu") (tenting (front no) (back no)) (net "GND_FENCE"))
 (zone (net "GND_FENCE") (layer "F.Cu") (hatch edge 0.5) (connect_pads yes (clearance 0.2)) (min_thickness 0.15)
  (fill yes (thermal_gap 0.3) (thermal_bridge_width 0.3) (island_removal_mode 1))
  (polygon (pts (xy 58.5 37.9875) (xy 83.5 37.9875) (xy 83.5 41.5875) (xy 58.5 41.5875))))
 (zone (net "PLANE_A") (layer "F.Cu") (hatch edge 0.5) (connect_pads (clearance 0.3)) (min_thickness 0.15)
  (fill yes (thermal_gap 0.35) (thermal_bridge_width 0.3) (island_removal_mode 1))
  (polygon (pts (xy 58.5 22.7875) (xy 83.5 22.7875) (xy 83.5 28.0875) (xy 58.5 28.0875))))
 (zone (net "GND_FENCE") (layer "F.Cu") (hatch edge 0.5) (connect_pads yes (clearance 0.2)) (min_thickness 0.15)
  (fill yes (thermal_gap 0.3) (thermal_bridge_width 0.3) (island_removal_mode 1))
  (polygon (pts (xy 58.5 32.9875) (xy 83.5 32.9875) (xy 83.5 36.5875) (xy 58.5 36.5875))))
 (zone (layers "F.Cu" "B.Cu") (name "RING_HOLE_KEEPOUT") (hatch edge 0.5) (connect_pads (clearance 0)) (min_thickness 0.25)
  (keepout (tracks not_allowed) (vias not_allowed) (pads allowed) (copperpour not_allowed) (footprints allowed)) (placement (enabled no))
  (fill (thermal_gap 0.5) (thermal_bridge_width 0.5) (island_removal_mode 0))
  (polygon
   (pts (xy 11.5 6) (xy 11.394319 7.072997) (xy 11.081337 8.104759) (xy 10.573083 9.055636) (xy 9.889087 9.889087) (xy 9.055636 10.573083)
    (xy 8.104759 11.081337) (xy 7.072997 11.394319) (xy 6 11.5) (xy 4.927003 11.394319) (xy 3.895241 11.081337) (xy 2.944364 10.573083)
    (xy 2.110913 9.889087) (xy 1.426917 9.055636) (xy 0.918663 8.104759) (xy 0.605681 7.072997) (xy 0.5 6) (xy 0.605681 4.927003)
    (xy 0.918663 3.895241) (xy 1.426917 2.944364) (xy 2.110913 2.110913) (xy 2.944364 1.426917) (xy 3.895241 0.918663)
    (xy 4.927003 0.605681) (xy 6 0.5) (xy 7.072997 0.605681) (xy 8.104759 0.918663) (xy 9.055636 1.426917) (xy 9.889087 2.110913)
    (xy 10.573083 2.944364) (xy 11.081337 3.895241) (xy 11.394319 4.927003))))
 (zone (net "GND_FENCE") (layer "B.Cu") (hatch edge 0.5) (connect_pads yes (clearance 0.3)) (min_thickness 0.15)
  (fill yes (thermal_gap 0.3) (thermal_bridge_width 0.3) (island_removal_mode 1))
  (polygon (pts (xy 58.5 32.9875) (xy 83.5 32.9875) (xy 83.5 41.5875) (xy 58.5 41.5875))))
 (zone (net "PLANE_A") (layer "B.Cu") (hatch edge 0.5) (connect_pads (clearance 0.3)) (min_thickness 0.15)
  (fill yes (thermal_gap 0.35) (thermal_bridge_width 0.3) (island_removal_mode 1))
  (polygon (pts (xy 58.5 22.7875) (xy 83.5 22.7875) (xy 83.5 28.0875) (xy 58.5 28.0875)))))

